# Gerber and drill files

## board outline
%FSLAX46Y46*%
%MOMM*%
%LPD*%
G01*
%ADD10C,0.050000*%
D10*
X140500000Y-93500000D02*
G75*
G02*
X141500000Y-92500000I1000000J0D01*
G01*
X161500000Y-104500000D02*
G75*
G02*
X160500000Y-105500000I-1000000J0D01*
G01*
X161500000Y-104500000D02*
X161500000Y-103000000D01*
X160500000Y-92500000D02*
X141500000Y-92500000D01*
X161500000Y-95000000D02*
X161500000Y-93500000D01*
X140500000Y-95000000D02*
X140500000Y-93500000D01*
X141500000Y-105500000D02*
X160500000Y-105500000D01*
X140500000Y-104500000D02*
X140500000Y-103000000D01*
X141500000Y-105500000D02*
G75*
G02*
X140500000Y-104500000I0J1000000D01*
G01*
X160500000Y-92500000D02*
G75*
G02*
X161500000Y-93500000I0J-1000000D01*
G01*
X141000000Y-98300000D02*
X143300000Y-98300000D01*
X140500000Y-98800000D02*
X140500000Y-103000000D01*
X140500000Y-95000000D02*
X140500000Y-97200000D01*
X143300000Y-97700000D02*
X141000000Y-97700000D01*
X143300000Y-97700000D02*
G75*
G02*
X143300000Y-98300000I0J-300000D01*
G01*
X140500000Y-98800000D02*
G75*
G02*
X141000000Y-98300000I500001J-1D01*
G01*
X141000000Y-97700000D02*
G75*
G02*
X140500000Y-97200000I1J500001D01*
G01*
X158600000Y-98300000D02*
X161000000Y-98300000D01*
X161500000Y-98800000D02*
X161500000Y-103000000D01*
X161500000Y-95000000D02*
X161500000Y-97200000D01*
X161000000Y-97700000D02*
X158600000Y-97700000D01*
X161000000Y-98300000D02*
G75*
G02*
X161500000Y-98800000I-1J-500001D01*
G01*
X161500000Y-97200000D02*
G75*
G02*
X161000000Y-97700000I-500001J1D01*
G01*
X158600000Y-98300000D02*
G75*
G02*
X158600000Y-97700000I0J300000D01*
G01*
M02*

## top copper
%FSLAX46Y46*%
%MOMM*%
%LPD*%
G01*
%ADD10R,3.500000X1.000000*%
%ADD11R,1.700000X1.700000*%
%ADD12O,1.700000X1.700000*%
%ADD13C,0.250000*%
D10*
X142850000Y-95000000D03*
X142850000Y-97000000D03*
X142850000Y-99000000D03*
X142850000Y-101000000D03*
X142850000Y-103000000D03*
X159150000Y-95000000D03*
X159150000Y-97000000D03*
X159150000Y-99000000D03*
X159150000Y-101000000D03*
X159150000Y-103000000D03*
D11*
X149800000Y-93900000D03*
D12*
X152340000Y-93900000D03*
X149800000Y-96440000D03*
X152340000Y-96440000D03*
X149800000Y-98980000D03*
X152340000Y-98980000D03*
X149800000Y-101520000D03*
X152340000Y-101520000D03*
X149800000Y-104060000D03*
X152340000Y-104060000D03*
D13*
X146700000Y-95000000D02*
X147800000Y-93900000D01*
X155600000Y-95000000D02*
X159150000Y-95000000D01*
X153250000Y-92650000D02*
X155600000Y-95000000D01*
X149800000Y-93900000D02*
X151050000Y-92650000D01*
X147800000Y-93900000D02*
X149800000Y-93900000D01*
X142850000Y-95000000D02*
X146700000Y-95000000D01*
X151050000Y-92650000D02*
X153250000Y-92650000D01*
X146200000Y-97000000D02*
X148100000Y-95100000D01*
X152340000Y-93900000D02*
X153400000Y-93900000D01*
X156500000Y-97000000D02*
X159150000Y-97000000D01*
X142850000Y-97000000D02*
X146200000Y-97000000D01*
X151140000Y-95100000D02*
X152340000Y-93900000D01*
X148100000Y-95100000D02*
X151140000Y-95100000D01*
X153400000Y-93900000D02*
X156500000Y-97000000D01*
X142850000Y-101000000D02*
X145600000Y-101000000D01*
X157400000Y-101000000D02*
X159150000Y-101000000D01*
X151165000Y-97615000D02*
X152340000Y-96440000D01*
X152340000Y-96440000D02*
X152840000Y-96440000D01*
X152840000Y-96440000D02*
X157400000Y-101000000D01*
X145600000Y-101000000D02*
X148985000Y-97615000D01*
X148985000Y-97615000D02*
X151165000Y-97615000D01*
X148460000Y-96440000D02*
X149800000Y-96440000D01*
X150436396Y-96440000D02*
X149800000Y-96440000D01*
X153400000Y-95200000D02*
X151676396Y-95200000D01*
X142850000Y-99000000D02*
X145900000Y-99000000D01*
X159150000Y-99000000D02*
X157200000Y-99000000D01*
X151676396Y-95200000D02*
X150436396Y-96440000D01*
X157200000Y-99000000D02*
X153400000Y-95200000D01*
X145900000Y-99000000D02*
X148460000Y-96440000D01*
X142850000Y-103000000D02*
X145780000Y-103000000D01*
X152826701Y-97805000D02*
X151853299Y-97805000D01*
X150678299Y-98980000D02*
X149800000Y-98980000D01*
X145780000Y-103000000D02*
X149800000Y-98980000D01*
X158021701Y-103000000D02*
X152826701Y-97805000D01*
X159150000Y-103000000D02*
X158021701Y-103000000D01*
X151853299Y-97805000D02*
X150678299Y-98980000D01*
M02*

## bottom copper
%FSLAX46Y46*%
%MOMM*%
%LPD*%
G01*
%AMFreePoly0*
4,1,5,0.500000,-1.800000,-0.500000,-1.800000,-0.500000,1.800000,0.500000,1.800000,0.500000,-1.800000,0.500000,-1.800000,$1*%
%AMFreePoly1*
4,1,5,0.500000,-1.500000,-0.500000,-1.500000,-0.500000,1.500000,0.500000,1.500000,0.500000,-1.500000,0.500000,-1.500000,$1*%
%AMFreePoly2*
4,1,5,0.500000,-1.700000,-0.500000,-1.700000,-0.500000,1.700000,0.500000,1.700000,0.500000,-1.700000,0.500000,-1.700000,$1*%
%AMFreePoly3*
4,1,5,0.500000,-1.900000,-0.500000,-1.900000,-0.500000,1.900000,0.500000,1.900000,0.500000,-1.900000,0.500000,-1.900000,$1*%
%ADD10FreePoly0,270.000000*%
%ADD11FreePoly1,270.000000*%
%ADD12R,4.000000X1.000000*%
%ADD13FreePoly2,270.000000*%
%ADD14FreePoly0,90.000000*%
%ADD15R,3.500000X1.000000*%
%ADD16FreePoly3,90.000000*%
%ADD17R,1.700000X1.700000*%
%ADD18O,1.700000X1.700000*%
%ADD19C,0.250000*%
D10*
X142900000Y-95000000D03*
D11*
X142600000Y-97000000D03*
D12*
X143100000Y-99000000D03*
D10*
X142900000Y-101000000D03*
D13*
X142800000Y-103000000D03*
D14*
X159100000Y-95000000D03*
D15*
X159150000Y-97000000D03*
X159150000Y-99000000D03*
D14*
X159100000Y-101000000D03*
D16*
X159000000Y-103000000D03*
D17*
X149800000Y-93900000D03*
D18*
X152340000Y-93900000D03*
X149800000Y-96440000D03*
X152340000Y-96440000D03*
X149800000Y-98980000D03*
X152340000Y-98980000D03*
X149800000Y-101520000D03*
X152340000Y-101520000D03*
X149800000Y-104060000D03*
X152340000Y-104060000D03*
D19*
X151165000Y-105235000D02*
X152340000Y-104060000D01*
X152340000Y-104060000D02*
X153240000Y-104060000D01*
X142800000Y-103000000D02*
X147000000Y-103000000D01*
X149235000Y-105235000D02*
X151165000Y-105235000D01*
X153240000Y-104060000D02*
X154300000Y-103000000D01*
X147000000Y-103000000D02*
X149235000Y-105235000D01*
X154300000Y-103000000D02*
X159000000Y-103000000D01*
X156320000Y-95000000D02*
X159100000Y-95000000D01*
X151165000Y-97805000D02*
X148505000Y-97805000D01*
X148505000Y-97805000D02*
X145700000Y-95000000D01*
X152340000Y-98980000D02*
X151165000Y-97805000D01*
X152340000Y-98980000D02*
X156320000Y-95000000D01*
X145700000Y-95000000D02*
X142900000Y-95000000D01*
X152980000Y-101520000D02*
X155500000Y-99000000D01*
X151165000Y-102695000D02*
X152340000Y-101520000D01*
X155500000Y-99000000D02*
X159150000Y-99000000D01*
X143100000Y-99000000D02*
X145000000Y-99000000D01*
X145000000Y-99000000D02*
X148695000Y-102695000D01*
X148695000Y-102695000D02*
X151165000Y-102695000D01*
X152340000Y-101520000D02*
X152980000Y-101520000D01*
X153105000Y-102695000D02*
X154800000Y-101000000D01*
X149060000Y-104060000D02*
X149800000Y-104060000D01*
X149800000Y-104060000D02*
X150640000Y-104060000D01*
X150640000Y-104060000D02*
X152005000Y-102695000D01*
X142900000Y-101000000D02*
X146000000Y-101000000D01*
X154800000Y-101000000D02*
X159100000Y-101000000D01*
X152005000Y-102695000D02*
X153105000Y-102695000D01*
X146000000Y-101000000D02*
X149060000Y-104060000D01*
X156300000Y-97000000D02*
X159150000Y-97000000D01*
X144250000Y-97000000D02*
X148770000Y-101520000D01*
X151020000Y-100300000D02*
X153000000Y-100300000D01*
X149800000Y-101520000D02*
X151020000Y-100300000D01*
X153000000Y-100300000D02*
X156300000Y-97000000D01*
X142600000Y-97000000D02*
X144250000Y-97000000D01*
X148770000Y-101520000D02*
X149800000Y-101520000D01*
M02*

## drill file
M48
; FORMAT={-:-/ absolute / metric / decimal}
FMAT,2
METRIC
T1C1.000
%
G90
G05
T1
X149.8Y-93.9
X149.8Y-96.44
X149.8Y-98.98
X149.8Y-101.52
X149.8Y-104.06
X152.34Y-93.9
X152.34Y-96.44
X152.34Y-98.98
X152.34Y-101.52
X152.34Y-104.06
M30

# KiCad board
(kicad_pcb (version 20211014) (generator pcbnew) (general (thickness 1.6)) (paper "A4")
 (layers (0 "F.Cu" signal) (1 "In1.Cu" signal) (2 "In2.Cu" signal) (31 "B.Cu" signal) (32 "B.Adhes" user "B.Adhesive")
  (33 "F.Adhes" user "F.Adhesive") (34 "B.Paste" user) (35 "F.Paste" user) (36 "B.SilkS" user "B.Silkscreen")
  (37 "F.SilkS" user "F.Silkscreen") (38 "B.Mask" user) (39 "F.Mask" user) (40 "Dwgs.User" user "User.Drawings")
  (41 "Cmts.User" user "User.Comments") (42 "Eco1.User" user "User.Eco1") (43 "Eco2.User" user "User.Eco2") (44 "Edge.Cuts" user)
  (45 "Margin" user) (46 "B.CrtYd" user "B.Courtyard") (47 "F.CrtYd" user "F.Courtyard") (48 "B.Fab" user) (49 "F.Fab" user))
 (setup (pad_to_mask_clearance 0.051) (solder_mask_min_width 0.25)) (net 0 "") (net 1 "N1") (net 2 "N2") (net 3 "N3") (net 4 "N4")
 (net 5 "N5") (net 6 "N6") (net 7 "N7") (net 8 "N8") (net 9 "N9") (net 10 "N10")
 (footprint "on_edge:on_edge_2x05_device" (layer "F.Cu") (at 140.5 99 -90)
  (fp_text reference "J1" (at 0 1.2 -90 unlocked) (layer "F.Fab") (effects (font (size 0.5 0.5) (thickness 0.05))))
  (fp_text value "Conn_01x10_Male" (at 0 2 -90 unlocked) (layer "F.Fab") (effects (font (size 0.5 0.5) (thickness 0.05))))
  (fp_line (start -0.7 -0.5) (end -0.7 -2.8) (layer "Edge.Cuts") (width 0.05))
  (fp_line (start -0.2 0) (end 4 0) (layer "Edge.Cuts") (width 0.05))
  (fp_line (start -4 0) (end -1.8 0) (layer "Edge.Cuts") (width 0.05))
  (fp_line (start -1.3 -2.8) (end -1.3 -0.5) (layer "Edge.Cuts") (width 0.05))
  (fp_arc (start -1.3 -2.8) (mid -1 -3.1) (end -0.7 -2.8) (layer "Edge.Cuts") (width 0.05))
  (fp_arc (start -0.2 0) (mid -0.553553 -0.146447) (end -0.7 -0.5) (layer "Edge.Cuts") (width 0.05))
  (fp_arc (start -1.3 -0.5) (mid -1.446447 -0.146447) (end -1.8 0) (layer "Edge.Cuts") (width 0.05))
  (pad "1" smd rect (at -4 -2.35 90) (size 1 3.5) (layers "F.Cu" "F.Mask") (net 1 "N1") (zone_connect 0))
  (pad "2" smd rect (at -2 -2.35 270) (size 1 3.5) (layers "F.Cu" "F.Mask") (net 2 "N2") (zone_connect 0))
  (pad "3" smd rect (at 0 -2.35 270) (size 1 3.5) (layers "F.Cu" "F.Mask") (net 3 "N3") (zone_connect 0))
  (pad "4" smd rect (at 2 -2.35 90) (size 1 3.5) (layers "F.Cu" "F.Mask") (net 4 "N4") (zone_connect 0))
  (pad "5" smd rect (at 4 -2.35 90) (size 1 3.5) (layers "F.Cu" "F.Mask") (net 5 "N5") (zone_connect 0))
  (pad "6" smd custom (at -4 -2.4 270) (size 1 3.6) (layers "B.Cu" "B.Mask") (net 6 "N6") (zone_connect 0)
   (options (clearance outline) (anchor rect)) (primitives))
  (pad "7" smd custom (at -2 -2.1 270) (size 1 3) (layers "B.Cu" "B.Mask") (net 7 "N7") (zone_connect 0)
   (options (clearance outline) (anchor rect)) (primitives))
  (pad "8" smd rect (at 0 -2.6 270) (size 1 4) (layers "B.Cu" "B.Mask") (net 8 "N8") (zone_connect 0))
  (pad "9" smd custom (at 2 -2.4 270) (size 1 3.6) (layers "B.Cu" "B.Mask") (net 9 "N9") (zone_connect 0)
   (options (clearance outline) (anchor rect)) (primitives))
  (pad "10" smd custom (at 4 -2.3 270) (size 1 3.4) (layers "B.Cu" "B.Mask") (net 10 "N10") (zone_connect 0)
   (options (clearance outline) (anchor rect)) (primitives)))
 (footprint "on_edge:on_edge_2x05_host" (layer "F.Cu") (at 161.5 99 -90)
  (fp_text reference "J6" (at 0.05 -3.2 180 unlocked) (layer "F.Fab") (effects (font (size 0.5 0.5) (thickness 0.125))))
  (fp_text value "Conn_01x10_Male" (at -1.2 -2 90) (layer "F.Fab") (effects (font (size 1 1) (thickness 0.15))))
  (fp_line (start -0.7 2.9) (end -0.7 0.5) (layer "Edge.Cuts") (width 0.05))
  (fp_line (start -0.2 0) (end 4 0) (layer "Edge.Cuts") (width 0.05))
  (fp_line (start -4 0) (end -1.8 0) (layer "Edge.Cuts") (width 0.05))
  (fp_line (start -1.3 0.5) (end -1.3 2.9) (layer "Edge.Cuts") (width 0.05))
  (fp_arc (start -0.7 0.5) (mid -0.553553 0.146447) (end -0.2 0) (layer "Edge.Cuts") (width 0.05))
  (fp_arc (start -1.8 0) (mid -1.446447 0.146447) (end -1.3 0.5) (layer "Edge.Cuts") (width 0.05))
  (fp_arc (start -0.7 2.9) (mid -1 3.2) (end -1.3 2.9) (layer "Edge.Cuts") (width 0.05))
  (pad "1" smd rect (at -4 2.35 270) (size 1 3.5) (layers "F.Cu" "F.Mask") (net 1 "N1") (zone_connect 0))
  (pad "2" smd rect (at -2 2.35 270) (size 1 3.5) (layers "F.Cu" "F.Mask") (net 2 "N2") (zone_connect 0))
  (pad "3" smd rect (at 0 2.35 270) (size 1 3.5) (layers "F.Cu" "F.Mask") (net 3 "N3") (zone_connect 0))
  (pad "4" smd rect (at 2 2.35 270) (size 1 3.5) (layers "F.Cu" "F.Mask") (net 4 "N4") (zone_connect 0))
  (pad "5" smd rect (at 4 2.35 270) (size 1 3.5) (layers "F.Cu" "F.Mask") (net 5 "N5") (zone_connect 0))
  (pad "6" smd custom (at -4 2.4 90) (size 1 3.6) (layers "B.Cu" "B.Mask") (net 6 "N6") (zone_connect 0)
   (options (clearance outline) (anchor rect)) (primitives))
  (pad "7" smd rect (at -2 2.35 90) (size 1 3.5) (layers "B.Cu" "B.Mask") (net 7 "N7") (zone_connect 0))
  (pad "8" smd rect (at 0 2.35 90) (size 1 3.5) (layers "B.Cu" "B.Mask") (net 8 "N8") (zone_connect 0))
  (pad "9" smd custom (at 2 2.4 90) (size 1 3.6) (layers "B.Cu" "B.Mask") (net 9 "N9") (zone_connect 0)
   (options (clearance outline) (anchor rect)) (primitives))
  (pad "10" smd custom (at 4 2.5 90) (size 1 3.8) (layers "B.Cu" "B.Mask") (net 10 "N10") (zone_connect 0)
   (options (clearance outline) (anchor rect)) (primitives)))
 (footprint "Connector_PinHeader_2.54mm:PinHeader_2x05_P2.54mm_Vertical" (layer "F.Cu") (at 149.8 93.9)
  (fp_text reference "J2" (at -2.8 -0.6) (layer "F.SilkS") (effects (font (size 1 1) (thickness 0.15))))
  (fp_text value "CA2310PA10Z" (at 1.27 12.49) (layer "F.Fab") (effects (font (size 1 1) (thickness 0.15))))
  (pad "1" thru_hole rect (at 0 0) (size 1.7 1.7) (drill 1) (layers *.Cu *.Mask) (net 1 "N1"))
  (pad "2" thru_hole oval (at 2.54 0) (size 1.7 1.7) (drill 1) (layers *.Cu *.Mask) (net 2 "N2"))
  (pad "3" thru_hole oval (at 0 2.54) (size 1.7 1.7) (drill 1) (layers *.Cu *.Mask) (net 3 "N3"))
  (pad "4" thru_hole oval (at 2.54 2.54) (size 1.7 1.7) (drill 1) (layers *.Cu *.Mask) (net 4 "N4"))
  (pad "5" thru_hole oval (at 0 5.08) (size 1.7 1.7) (drill 1) (layers *.Cu *.Mask) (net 5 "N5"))
  (pad "6" thru_hole oval (at 2.54 5.08) (size 1.7 1.7) (drill 1) (layers *.Cu *.Mask) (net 6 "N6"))
  (pad "7" thru_hole oval (at 0 7.62) (size 1.7 1.7) (drill 1) (layers *.Cu *.Mask) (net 7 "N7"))
  (pad "8" thru_hole oval (at 2.54 7.62) (size 1.7 1.7) (drill 1) (layers *.Cu *.Mask) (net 8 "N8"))
  (pad "9" thru_hole oval (at 0 10.16) (size 1.7 1.7) (drill 1) (layers *.Cu *.Mask) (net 9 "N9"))
  (pad "10" thru_hole oval (at 2.54 10.16) (size 1.7 1.7) (drill 1) (layers *.Cu *.Mask) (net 10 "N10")))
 (gr_arc (start 140.5 93.5) (mid 140.792893 92.792893) (end 141.5 92.5) (layer "Edge.Cuts") (width 0.05))
 (gr_arc (start 161.5 104.5) (mid 161.207107 105.207107) (end 160.5 105.5) (layer "Edge.Cuts") (width 0.05))
 (gr_line (start 161.5 104.5) (end 161.5 103) (layer "Edge.Cuts") (width 0.05))
 (gr_line (start 160.5 92.5) (end 141.5 92.5) (layer "Edge.Cuts") (width 0.05))
 (gr_line (start 161.5 95) (end 161.5 93.5) (layer "Edge.Cuts") (width 0.05))
 (gr_line (start 140.5 95) (end 140.5 93.5) (layer "Edge.Cuts") (width 0.05))
 (gr_line (start 141.5 105.5) (end 160.5 105.5) (layer "Edge.Cuts") (width 0.05))
 (gr_line (start 140.5 104.5) (end 140.5 103) (layer "Edge.Cuts") (width 0.05))
 (gr_arc (start 141.5 105.5) (mid 140.792893 105.207107) (end 140.5 104.5) (layer "Edge.Cuts") (width 0.05))
 (gr_arc (start 160.5 92.5) (mid 161.207107 92.792893) (end 161.5 93.5) (layer "Edge.Cuts") (width 0.05))
 (segment (start 146.7 95) (end 147.8 93.9) (width 0.25) (layer "F.Cu") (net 1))
 (segment (start 155.6 95) (end 159.15 95) (width 0.25) (layer "F.Cu") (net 1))
 (segment (start 153.25 92.65) (end 155.6 95) (width 0.25) (layer "F.Cu") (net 1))
 (segment (start 149.8 93.9) (end 151.05 92.65) (width 0.25) (layer "F.Cu") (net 1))
 (segment (start 147.8 93.9) (end 149.8 93.9) (width 0.25) (layer "F.Cu") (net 1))
 (segment (start 142.85 95) (end 146.7 95) (width 0.25) (layer "F.Cu") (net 1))
 (segment (start 151.05 92.65) (end 153.25 92.65) (width 0.25) (layer "F.Cu") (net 1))
 (segment (start 146.2 97) (end 148.1 95.1) (width 0.25) (layer "F.Cu") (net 2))
 (segment (start 152.34 93.9) (end 153.4 93.9) (width 0.25) (layer "F.Cu") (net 2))
 (segment (start 156.5 97) (end 159.15 97) (width 0.25) (layer "F.Cu") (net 2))
 (segment (start 142.85 97) (end 146.2 97) (width 0.25) (layer "F.Cu") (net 2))
 (segment (start 151.14 95.1) (end 152.34 93.9) (width 0.25) (layer "F.Cu") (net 2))
 (segment (start 148.1 95.1) (end 151.14 95.1) (width 0.25) (layer "F.Cu") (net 2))
 (segment (start 153.4 93.9) (end 156.5 97) (width 0.25) (layer "F.Cu") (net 2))
 (segment (start 142.85 101) (end 145.6 101) (width 0.25) (layer "F.Cu") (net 4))
 (segment (start 157.4 101) (end 159.15 101) (width 0.25) (layer "F.Cu") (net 4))
 (segment (start 151.165 97.615) (end 152.34 96.44) (width 0.25) (layer "F.Cu") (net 4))
 (segment (start 152.34 96.44) (end 152.84 96.44) (width 0.25) (layer "F.Cu") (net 4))
 (segment (start 152.84 96.44) (end 157.4 101) (width 0.25) (layer "F.Cu") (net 4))
 (segment (start 145.6 101) (end 148.985 97.615) (width 0.25) (layer "F.Cu") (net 4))
 (segment (start 148.985 97.615) (end 151.165 97.615) (width 0.25) (layer "F.Cu") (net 4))
 (segment (start 148.46 96.44) (end 149.8 96.44) (width 0.25) (layer "F.Cu") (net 3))
 (segment (start 150.436396 96.44) (end 149.8 96.44) (width 0.25) (layer "F.Cu") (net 3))
 (segment (start 153.4 95.2) (end 151.676396 95.2) (width 0.25) (layer "F.Cu") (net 3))
 (segment (start 142.85 99) (end 145.9 99) (width 0.25) (layer "F.Cu") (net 3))
 (segment (start 159.15 99) (end 157.2 99) (width 0.25) (layer "F.Cu") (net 3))
 (segment (start 151.676396 95.2) (end 150.436396 96.44) (width 0.25) (layer "F.Cu") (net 3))
 (segment (start 157.2 99) (end 153.4 95.2) (width 0.25) (layer "F.Cu") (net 3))
 (segment (start 145.9 99) (end 148.46 96.44) (width 0.25) (layer "F.Cu") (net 3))
 (segment (start 151.165 105.235) (end 152.34 104.06) (width 0.25) (layer "B.Cu") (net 10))
 (segment (start 152.34 104.06) (end 153.24 104.06) (width 0.25) (layer "B.Cu") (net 10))
 (segment (start 142.8 103) (end 147 103) (width 0.25) (layer "B.Cu") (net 10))
 (segment (start 149.235 105.235) (end 151.165 105.235) (width 0.25) (layer "B.Cu") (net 10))
 (segment (start 153.24 104.06) (end 154.3 103) (width 0.25) (layer "B.Cu") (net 10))
 (segment (start 147 103) (end 149.235 105.235) (width 0.25) (layer "B.Cu") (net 10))
 (segment (start 154.3 103) (end 159 103) (width 0.25) (layer "B.Cu") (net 10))
 (segment (start 156.32 95) (end 159.1 95) (width 0.25) (layer "B.Cu") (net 6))
 (segment (start 151.165 97.805) (end 148.505 97.805) (width 0.25) (layer "B.Cu") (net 6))
 (segment (start 148.505 97.805) (end 145.7 95) (width 0.25) (layer "B.Cu") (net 6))
 (segment (start 152.34 98.98) (end 151.165 97.805) (width 0.25) (layer "B.Cu") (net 6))
 (segment (start 152.34 98.98) (end 156.32 95) (width 0.25) (layer "B.Cu") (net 6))
 (segment (start 145.7 95) (end 142.9 95) (width 0.25) (layer "B.Cu") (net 6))
 (segment (start 152.98 101.52) (end 155.5 99) (width 0.25) (layer "B.Cu") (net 8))
 (segment (start 151.165 102.695) (end 152.34 101.52) (width 0.25) (layer "B.Cu") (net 8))
 (segment (start 155.5 99) (end 159.15 99) (width 0.25) (layer "B.Cu") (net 8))
 (segment (start 143.1 99) (end 145 99) (width 0.25) (layer "B.Cu") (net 8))
 (segment (start 145 99) (end 148.695 102.695) (width 0.25) (layer "B.Cu") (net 8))
 (segment (start 148.695 102.695) (end 151.165 102.695) (width 0.25) (layer "B.Cu") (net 8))
 (segment (start 152.34 101.52) (end 152.98 101.52) (width 0.25) (layer "B.Cu") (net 8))
 (segment (start 153.105 102.695) (end 154.8 101) (width 0.25) (layer "B.Cu") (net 9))
 (segment (start 149.06 104.06) (end 149.8 104.06) (width 0.25) (layer "B.Cu") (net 9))
 (segment (start 149.8 104.06) (end 150.64 104.06) (width 0.25) (layer "B.Cu") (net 9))
 (segment (start 150.64 104.06) (end 152.005 102.695) (width 0.25) (layer "B.Cu") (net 9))
 (segment (start 142.9 101) (end 146 101) (width 0.25) (layer "B.Cu") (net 9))
 (segment (start 154.8 101) (end 159.1 101) (width 0.25) (layer "B.Cu") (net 9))
 (segment (start 152.005 102.695) (end 153.105 102.695) (width 0.25) (layer "B.Cu") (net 9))
 (segment (start 146 101) (end 149.06 104.06) (width 0.25) (layer "B.Cu") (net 9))
 (segment (start 156.3 97) (end 159.15 97) (width 0.25) (layer "B.Cu") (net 7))
 (segment (start 144.25 97) (end 148.77 101.52) (width 0.25) (layer "B.Cu") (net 7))
 (segment (start 151.02 100.3) (end 153 100.3) (width 0.25) (layer "B.Cu") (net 7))
 (segment (start 149.8 101.52) (end 151.02 100.3) (width 0.25) (layer "B.Cu") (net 7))
 (segment (start 153 100.3) (end 156.3 97) (width 0.25) (layer "B.Cu") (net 7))
 (segment (start 142.6 97) (end 144.25 97) (width 0.25) (layer "B.Cu") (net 7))
 (segment (start 148.77 101.52) (end 149.8 101.52) (width 0.25) (layer "B.Cu") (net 7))
 (segment (start 142.85 103) (end 145.78 103) (width 0.25) (layer "F.Cu") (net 5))
 (segment (start 152.826701 97.805) (end 151.853299 97.805) (width 0.25) (layer "F.Cu") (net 5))
 (segment (start 150.678299 98.98) (end 149.8 98.98) (width 0.25) (layer "F.Cu") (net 5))
 (segment (start 145.78 103) (end 149.8 98.98) (width 0.25) (layer "F.Cu") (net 5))
 (segment (start 158.021701 103) (end 152.826701 97.805) (width 0.25) (layer "F.Cu") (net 5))
 (segment (start 159.15 103) (end 158.021701 103) (width 0.25) (layer "F.Cu") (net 5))
 (segment (start 151.853299 97.805) (end 150.678299 98.98) (width 0.25) (layer "F.Cu") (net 5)))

